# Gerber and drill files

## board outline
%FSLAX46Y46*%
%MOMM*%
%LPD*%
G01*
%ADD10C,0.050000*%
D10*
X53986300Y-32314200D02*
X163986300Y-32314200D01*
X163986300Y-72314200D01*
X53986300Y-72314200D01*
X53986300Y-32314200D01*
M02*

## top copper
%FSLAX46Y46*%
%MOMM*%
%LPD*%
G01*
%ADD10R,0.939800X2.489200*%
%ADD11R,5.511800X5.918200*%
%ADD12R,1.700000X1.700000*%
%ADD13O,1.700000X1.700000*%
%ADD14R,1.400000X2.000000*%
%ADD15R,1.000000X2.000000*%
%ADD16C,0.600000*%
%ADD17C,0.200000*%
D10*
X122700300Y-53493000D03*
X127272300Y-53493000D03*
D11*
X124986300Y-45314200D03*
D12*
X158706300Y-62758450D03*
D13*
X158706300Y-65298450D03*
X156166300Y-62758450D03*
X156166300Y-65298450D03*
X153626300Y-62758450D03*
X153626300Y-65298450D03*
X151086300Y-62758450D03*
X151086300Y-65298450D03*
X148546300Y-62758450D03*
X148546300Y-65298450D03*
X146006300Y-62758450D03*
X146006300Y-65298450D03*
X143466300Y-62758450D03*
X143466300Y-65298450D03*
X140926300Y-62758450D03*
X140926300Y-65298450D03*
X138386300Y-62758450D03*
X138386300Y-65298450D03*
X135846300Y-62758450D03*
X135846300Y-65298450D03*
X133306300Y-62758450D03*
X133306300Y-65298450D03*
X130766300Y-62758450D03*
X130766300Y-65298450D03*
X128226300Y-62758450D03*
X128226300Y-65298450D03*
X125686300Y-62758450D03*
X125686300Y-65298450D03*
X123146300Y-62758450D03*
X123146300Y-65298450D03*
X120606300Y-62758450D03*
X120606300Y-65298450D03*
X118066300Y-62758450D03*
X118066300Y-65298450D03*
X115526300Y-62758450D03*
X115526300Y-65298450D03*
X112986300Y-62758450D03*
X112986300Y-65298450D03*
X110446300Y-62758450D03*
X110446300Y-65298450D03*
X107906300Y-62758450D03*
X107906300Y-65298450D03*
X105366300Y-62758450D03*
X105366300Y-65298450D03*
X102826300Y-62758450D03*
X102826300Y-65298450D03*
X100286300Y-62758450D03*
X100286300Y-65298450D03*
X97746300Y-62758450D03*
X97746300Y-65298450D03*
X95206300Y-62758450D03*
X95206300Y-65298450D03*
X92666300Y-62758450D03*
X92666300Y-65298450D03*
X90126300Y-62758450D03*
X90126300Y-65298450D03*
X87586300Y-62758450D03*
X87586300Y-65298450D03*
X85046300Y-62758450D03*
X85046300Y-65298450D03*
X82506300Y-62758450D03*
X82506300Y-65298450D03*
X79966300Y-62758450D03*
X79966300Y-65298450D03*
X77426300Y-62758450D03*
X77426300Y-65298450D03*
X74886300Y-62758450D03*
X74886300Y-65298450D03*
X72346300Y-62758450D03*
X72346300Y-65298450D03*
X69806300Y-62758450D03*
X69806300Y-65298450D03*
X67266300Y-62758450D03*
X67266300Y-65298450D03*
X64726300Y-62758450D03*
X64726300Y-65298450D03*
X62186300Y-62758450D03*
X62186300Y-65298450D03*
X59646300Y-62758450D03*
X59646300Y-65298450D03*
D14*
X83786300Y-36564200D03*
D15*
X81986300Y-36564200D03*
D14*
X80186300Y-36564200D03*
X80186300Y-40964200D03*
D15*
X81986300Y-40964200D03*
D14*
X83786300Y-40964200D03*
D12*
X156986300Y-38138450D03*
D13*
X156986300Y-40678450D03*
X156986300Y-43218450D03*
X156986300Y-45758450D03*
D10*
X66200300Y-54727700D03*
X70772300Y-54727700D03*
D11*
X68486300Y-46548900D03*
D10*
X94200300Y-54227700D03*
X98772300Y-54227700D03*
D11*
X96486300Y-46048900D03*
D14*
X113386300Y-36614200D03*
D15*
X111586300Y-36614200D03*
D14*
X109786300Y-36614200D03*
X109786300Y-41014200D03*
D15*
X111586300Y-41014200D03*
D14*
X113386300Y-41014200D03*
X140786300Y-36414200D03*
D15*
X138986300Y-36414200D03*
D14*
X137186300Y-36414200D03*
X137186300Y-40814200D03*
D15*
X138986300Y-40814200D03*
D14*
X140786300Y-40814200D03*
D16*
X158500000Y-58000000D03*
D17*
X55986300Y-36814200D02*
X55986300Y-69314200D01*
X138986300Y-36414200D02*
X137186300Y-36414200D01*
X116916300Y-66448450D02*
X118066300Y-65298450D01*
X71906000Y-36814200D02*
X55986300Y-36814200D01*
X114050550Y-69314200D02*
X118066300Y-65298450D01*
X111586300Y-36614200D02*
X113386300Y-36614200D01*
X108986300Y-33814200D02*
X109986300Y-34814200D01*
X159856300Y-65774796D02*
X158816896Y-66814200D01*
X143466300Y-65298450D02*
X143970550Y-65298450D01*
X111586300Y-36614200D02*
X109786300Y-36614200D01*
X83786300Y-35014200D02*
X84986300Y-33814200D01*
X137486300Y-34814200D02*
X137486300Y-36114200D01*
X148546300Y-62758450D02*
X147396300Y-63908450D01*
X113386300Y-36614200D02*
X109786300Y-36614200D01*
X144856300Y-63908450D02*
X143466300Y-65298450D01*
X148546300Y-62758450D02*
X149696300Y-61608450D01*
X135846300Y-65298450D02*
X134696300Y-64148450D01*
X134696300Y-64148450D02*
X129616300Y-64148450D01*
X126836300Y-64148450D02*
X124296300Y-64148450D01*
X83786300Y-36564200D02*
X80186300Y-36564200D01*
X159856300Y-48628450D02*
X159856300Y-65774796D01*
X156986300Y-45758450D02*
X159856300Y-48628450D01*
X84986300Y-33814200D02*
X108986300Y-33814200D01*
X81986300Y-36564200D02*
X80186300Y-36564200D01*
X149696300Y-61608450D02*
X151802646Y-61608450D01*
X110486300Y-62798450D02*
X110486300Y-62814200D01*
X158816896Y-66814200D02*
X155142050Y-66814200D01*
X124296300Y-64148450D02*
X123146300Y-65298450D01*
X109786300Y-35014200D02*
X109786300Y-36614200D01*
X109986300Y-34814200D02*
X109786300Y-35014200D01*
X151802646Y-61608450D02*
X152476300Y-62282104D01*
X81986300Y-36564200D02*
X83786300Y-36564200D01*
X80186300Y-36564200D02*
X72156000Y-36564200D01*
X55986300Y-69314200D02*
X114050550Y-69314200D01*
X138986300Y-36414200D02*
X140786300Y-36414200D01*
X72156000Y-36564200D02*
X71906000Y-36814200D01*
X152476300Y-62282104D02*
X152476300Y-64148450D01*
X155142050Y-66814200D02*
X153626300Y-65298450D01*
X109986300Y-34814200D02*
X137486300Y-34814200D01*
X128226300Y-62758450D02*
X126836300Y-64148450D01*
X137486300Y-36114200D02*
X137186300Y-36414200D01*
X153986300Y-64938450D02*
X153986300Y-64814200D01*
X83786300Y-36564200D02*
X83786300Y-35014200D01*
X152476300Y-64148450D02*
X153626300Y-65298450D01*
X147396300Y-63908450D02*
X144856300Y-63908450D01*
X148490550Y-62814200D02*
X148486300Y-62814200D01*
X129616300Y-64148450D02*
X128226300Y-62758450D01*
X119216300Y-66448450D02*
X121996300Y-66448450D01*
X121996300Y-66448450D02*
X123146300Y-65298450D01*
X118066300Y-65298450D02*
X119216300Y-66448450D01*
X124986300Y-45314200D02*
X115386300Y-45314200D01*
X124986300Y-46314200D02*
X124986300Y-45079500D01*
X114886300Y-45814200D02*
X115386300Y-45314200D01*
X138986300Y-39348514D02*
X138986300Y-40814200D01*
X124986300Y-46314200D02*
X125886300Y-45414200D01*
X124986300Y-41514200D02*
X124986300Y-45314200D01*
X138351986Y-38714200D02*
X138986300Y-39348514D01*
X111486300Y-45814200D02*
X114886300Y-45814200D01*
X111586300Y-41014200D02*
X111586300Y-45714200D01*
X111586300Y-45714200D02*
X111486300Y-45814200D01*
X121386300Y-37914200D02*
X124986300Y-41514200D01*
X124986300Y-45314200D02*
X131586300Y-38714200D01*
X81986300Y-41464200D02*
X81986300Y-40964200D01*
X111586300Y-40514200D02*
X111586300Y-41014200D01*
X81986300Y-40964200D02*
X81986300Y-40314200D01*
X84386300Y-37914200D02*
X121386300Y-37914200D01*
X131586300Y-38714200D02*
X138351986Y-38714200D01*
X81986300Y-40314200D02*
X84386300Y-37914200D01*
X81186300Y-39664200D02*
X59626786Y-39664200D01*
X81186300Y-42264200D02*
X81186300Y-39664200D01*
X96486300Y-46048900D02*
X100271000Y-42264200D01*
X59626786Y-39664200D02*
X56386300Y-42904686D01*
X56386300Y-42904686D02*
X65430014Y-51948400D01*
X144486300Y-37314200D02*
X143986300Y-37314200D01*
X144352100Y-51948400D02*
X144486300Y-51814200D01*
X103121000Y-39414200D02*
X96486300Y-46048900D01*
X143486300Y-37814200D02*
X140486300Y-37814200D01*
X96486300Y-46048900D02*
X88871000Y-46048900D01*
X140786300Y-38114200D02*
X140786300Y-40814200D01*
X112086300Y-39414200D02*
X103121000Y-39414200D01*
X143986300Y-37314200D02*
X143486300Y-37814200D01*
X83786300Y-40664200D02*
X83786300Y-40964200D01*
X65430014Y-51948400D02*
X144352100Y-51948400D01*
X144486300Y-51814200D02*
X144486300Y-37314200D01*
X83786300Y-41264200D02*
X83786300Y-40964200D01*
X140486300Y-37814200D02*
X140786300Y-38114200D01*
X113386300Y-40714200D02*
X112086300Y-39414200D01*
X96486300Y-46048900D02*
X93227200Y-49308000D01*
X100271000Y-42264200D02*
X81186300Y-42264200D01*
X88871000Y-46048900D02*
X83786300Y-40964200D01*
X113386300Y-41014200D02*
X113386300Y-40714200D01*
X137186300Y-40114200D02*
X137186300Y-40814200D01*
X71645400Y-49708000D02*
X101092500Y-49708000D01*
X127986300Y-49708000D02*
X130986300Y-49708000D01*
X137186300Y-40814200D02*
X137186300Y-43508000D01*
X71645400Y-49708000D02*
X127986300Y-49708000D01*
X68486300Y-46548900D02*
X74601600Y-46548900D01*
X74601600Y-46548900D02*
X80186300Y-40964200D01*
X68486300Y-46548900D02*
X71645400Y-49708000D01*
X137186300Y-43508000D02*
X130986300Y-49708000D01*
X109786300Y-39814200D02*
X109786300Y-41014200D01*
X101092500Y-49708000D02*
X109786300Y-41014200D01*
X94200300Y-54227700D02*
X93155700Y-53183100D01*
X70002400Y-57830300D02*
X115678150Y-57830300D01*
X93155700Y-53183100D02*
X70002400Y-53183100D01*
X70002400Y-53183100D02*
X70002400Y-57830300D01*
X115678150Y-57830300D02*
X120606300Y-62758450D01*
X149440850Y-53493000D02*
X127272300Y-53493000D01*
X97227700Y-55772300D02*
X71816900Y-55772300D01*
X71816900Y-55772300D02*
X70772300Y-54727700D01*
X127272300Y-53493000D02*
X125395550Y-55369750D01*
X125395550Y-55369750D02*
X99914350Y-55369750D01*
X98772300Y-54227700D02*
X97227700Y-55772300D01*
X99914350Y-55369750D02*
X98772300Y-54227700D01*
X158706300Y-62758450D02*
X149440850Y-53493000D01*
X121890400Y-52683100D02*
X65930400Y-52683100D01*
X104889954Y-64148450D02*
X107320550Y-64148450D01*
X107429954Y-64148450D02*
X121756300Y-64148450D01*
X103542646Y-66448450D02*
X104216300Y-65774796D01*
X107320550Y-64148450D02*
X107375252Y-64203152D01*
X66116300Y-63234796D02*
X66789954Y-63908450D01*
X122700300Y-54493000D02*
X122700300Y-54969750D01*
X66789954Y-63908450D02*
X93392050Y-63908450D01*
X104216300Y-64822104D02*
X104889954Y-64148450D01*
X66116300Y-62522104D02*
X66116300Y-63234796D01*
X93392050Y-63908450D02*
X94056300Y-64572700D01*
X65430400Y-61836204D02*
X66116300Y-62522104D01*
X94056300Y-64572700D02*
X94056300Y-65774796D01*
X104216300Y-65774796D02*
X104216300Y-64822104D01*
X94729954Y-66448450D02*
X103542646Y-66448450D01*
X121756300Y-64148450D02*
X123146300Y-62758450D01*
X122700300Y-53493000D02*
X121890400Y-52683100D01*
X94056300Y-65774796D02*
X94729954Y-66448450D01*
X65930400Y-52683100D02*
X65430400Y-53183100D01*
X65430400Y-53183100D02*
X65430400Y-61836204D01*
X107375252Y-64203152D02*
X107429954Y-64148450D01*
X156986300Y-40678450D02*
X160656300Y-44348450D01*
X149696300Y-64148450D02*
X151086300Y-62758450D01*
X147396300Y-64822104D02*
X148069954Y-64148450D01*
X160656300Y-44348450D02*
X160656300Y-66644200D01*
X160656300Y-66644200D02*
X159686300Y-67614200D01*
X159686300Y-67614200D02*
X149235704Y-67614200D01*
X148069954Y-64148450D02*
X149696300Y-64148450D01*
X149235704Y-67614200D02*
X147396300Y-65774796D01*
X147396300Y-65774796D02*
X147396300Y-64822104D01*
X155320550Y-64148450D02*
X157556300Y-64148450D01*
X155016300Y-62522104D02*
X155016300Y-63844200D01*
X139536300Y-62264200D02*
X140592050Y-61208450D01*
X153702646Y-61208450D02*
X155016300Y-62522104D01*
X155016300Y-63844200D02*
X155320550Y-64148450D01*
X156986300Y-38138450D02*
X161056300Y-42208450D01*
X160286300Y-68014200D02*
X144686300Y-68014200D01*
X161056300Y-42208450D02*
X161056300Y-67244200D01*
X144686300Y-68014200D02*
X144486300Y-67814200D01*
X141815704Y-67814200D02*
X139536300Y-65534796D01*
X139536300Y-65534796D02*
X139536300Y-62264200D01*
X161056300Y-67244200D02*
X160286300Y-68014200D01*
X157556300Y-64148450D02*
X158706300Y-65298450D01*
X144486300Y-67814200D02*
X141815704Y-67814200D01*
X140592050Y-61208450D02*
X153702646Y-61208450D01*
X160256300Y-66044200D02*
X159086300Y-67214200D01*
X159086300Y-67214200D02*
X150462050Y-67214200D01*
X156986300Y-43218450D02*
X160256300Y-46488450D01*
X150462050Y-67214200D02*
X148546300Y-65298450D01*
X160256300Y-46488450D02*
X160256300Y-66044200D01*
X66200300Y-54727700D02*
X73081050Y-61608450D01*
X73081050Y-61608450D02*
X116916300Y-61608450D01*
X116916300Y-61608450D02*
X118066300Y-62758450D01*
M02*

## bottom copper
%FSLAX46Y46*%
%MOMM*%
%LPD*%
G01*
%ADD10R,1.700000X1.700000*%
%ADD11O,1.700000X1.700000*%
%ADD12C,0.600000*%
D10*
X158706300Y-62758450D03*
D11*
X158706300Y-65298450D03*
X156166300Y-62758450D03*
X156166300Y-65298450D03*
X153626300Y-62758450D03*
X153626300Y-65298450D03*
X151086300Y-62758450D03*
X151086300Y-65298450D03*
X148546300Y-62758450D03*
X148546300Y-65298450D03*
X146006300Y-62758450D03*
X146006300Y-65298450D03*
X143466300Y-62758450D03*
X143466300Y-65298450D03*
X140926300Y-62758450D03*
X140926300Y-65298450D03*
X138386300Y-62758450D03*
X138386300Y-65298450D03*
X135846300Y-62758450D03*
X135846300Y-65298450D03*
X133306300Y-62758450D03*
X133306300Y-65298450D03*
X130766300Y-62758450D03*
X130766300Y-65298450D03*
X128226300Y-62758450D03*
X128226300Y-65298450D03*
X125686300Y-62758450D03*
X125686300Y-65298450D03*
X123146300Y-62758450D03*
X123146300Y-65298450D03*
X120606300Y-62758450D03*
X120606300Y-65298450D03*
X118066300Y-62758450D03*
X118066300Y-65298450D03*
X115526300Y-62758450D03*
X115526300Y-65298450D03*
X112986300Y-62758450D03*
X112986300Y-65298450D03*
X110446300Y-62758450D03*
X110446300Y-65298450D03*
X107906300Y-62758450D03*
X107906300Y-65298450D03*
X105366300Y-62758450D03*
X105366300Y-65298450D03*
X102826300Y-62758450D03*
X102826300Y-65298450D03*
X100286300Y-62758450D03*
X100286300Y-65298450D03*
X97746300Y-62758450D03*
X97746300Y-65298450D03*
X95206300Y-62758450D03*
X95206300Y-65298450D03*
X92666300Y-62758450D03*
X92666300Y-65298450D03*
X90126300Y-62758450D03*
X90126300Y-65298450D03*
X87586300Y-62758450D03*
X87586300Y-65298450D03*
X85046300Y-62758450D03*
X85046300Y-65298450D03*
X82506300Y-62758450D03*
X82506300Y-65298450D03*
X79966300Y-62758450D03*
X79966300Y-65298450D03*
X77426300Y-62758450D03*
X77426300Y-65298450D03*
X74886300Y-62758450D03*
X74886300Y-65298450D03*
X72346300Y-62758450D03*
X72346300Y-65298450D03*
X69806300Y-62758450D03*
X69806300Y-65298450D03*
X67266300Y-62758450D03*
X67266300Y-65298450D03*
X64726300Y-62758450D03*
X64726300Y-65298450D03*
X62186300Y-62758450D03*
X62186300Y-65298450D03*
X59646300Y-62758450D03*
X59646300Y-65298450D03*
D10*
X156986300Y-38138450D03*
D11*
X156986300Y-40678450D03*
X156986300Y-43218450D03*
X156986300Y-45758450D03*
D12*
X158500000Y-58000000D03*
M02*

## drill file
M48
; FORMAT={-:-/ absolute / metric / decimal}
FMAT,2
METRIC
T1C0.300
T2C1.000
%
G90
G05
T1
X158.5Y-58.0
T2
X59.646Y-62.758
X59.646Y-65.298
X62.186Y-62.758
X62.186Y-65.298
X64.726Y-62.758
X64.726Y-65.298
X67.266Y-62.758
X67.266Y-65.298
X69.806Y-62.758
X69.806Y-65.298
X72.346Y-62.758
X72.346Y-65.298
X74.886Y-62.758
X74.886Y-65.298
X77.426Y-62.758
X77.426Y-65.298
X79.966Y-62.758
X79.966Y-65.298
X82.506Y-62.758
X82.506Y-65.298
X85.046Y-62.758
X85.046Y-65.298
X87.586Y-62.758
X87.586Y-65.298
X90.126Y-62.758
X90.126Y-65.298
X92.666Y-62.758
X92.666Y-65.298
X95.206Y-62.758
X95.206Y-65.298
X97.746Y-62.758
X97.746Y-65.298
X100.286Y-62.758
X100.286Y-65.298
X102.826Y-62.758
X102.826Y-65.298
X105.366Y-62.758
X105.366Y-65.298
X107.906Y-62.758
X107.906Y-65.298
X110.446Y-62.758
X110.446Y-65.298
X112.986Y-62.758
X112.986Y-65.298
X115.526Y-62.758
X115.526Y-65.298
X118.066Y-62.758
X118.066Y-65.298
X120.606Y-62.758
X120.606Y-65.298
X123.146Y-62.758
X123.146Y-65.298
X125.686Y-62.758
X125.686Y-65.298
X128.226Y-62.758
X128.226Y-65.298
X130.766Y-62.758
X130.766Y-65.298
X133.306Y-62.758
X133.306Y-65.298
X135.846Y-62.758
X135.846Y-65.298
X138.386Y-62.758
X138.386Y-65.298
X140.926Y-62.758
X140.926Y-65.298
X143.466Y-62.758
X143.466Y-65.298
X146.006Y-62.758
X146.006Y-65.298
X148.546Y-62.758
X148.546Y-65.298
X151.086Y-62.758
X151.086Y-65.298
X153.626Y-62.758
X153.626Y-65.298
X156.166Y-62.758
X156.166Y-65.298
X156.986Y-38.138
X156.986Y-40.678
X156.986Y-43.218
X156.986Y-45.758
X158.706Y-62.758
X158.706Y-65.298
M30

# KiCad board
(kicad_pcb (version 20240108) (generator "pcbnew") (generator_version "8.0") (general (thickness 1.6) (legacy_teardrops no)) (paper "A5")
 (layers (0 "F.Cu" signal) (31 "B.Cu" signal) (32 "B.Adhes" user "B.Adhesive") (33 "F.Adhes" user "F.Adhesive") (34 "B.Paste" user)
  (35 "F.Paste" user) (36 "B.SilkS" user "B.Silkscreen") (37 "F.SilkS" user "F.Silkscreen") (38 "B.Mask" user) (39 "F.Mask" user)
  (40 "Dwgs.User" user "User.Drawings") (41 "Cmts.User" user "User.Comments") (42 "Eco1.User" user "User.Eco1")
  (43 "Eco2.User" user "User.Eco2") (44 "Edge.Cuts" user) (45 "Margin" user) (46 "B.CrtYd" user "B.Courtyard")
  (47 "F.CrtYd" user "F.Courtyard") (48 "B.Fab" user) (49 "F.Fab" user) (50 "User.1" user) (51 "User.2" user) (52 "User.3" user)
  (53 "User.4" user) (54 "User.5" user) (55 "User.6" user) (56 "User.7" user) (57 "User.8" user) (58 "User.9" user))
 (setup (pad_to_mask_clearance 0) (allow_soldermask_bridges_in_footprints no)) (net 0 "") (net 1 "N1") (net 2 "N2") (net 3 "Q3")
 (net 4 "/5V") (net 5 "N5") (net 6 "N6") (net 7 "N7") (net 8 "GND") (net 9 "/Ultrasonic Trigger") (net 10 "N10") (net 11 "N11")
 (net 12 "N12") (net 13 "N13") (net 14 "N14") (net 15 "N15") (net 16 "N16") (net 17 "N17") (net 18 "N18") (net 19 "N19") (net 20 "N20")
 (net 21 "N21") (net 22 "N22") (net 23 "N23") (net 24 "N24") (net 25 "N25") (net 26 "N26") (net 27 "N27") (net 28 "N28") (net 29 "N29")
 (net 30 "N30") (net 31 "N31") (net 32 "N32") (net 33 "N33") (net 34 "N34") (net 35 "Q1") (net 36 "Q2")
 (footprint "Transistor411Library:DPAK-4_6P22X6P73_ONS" (layer "F.Cu") (at 124.9863 47.0795)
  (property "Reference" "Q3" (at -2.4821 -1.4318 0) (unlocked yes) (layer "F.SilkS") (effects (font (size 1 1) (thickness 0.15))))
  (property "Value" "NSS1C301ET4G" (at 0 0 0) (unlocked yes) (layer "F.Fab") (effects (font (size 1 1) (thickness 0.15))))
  (pad "1" smd rect (at -2.286 6.4135) (size 0.9398 2.4892) (layers "F.Cu" "F.Paste" "F.Mask") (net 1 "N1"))
  (pad "2" smd rect (at 2.286 6.4135) (size 0.9398 2.4892) (layers "F.Cu" "F.Paste" "F.Mask") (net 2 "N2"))
  (pad "3" smd rect (at 0 -1.7653) (size 5.5118 5.9182) (layers "F.Cu" "F.Paste" "F.Mask") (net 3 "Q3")))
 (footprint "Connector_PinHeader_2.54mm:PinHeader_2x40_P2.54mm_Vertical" (layer "F.Cu") (at 158.7063 62.75845 -90)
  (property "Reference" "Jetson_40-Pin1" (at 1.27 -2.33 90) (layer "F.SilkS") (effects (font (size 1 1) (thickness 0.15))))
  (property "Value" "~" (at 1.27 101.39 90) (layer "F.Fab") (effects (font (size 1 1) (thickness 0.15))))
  (pad "1" thru_hole rect (at 0 0 270) (size 1.7 1.7) (drill 1) (layers "*.Cu" "*.Mask") (remove_unused_layers no) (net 2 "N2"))
  (pad "2" thru_hole oval (at 2.54 0 270) (size 1.7 1.7) (drill 1) (layers "*.Cu" "*.Mask") (remove_unused_layers no) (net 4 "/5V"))
  (pad "3" thru_hole oval (at 0 2.54 270) (size 1.7 1.7) (drill 1) (layers "*.Cu" "*.Mask") (remove_unused_layers no) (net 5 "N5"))
  (pad "4" thru_hole oval (at 2.54 2.54 270) (size 1.7 1.7) (drill 1) (layers "*.Cu" "*.Mask") (remove_unused_layers no) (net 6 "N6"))
  (pad "5" thru_hole oval (at 0 5.08 270) (size 1.7 1.7) (drill 1) (layers "*.Cu" "*.Mask") (remove_unused_layers no) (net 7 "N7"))
  (pad "6" thru_hole oval (at 2.54 5.08 270) (size 1.7 1.7) (drill 1) (layers "*.Cu" "*.Mask") (remove_unused_layers no) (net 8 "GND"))
  (pad "7" thru_hole oval (at 0 7.62 270) (size 1.7 1.7) (drill 1) (layers "*.Cu" "*.Mask") (remove_unused_layers no)
   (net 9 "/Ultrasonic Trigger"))
  (pad "8" thru_hole oval (at 2.54 7.62 270) (size 1.7 1.7) (drill 1) (layers "*.Cu" "*.Mask") (remove_unused_layers no) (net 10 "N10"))
  (pad "9" thru_hole oval (at 0 10.16 270) (size 1.7 1.7) (drill 1) (layers "*.Cu" "*.Mask") (remove_unused_layers no) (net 8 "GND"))
  (pad "10" thru_hole oval (at 2.54 10.16 270) (size 1.7 1.7) (drill 1) (layers "*.Cu" "*.Mask") (remove_unused_layers no) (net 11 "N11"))
  (pad "11" thru_hole oval (at 0 12.7 270) (size 1.7 1.7) (drill 1) (layers "*.Cu" "*.Mask") (remove_unused_layers no) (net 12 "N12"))
  (pad "12" thru_hole oval (at 2.54 12.7 270) (size 1.7 1.7) (drill 1) (layers "*.Cu" "*.Mask") (remove_unused_layers no) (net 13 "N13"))
  (pad "13" thru_hole oval (at 0 15.24 270) (size 1.7 1.7) (drill 1) (layers "*.Cu" "*.Mask") (remove_unused_layers no) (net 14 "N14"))
  (pad "14" thru_hole oval (at 2.54 15.24 270) (size 1.7 1.7) (drill 1) (layers "*.Cu" "*.Mask") (remove_unused_layers no) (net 8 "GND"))
  (pad "15" thru_hole oval (at 0 17.78 270) (size 1.7 1.7) (drill 1) (layers "*.Cu" "*.Mask") (remove_unused_layers no) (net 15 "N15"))
  (pad "16" thru_hole oval (at 2.54 17.78 270) (size 1.7 1.7) (drill 1) (layers "*.Cu" "*.Mask") (remove_unused_layers no) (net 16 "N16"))
  (pad "17" thru_hole oval (at 0 20.32 270) (size 1.7 1.7) (drill 1) (layers "*.Cu" "*.Mask") (remove_unused_layers no) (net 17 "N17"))
  (pad "18" thru_hole oval (at 2.54 20.32 270) (size 1.7 1.7) (drill 1) (layers "*.Cu" "*.Mask") (remove_unused_layers no) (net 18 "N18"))
  (pad "19" thru_hole oval (at 0 22.86 270) (size 1.7 1.7) (drill 1) (layers "*.Cu" "*.Mask") (remove_unused_layers no) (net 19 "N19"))
  (pad "20" thru_hole oval (at 2.54 22.86 270) (size 1.7 1.7) (drill 1) (layers "*.Cu" "*.Mask") (remove_unused_layers no) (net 8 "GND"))
  (pad "21" thru_hole oval (at 0 25.4 270) (size 1.7 1.7) (drill 1) (layers "*.Cu" "*.Mask") (remove_unused_layers no) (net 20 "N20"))
  (pad "22" thru_hole oval (at 2.54 25.4 270) (size 1.7 1.7) (drill 1) (layers "*.Cu" "*.Mask") (remove_unused_layers no) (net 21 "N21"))
  (pad "23" thru_hole oval (at 0 27.94 270) (size 1.7 1.7) (drill 1) (layers "*.Cu" "*.Mask") (remove_unused_layers no) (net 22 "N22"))
  (pad "24" thru_hole oval (at 2.54 27.94 270) (size 1.7 1.7) (drill 1) (layers "*.Cu" "*.Mask") (remove_unused_layers no) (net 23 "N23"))
  (pad "25" thru_hole oval (at 0 30.48 270) (size 1.7 1.7) (drill 1) (layers "*.Cu" "*.Mask") (remove_unused_layers no) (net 8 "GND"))
  (pad "26" thru_hole oval (at 2.54 30.48 270) (size 1.7 1.7) (drill 1) (layers "*.Cu" "*.Mask") (remove_unused_layers no) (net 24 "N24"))
  (pad "27" thru_hole oval (at 0 33.02 270) (size 1.7 1.7) (drill 1) (layers "*.Cu" "*.Mask") (remove_unused_layers no) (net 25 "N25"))
  (pad "28" thru_hole oval (at 2.54 33.02 270) (size 1.7 1.7) (drill 1) (layers "*.Cu" "*.Mask") (remove_unused_layers no) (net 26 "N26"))
  (pad "29" thru_hole oval (at 0 35.56 270) (size 1.7 1.7) (drill 1) (layers "*.Cu" "*.Mask") (remove_unused_layers no) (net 1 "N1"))
  (pad "30" thru_hole oval (at 2.54 35.56 270) (size 1.7 1.7) (drill 1) (layers "*.Cu" "*.Mask") (remove_unused_layers no) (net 8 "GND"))
  (pad "31" thru_hole oval (at 0 38.1 270) (size 1.7 1.7) (drill 1) (layers "*.Cu" "*.Mask") (remove_unused_layers no) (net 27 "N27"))
  (pad "32" thru_hole oval (at 2.54 38.1 270) (size 1.7 1.7) (drill 1) (layers "*.Cu" "*.Mask") (remove_unused_layers no) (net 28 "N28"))
  (pad "33" thru_hole oval (at 0 40.64 270) (size 1.7 1.7) (drill 1) (layers "*.Cu" "*.Mask") (remove_unused_layers no) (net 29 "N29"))
  (pad "34" thru_hole oval (at 2.54 40.64 270) (size 1.7 1.7) (drill 1) (layers "*.Cu" "*.Mask") (remove_unused_layers no) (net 8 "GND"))
  (pad "35" thru_hole oval (at 0 43.18 270) (size 1.7 1.7) (drill 1) (layers "*.Cu" "*.Mask") (remove_unused_layers no) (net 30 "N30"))
  (pad "36" thru_hole oval (at 2.54 43.18 270) (size 1.7 1.7) (drill 1) (layers "*.Cu" "*.Mask") (remove_unused_layers no) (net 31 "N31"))
  (pad "37" thru_hole oval (at 0 45.72 270) (size 1.7 1.7) (drill 1) (layers "*.Cu" "*.Mask") (remove_unused_layers no) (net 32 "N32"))
  (pad "38" thru_hole oval (at 2.54 45.72 270) (size 1.7 1.7) (drill 1) (layers "*.Cu" "*.Mask") (remove_unused_layers no) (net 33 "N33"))
  (pad "39" thru_hole oval (at 0 48.26 270) (size 1.7 1.7) (drill 1) (layers "*.Cu" "*.Mask") (remove_unused_layers no) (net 8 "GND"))
  (pad "40" thru_hole oval (at 2.54 48.26 270) (size 1.7 1.7) (drill 1) (layers "*.Cu" "*.Mask") (remove_unused_layers no) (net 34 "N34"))
  (pad "41" thru_hole oval (at 0 50.8 270) (size 1.7 1.7) (drill 1) (layers "*.Cu" "*.Mask") (remove_unused_layers no))
  (pad "42" thru_hole oval (at 2.54 50.8 270) (size 1.7 1.7) (drill 1) (layers "*.Cu" "*.Mask") (remove_unused_layers no))
  (pad "43" thru_hole oval (at 0 53.34 270) (size 1.7 1.7) (drill 1) (layers "*.Cu" "*.Mask") (remove_unused_layers no))
  (pad "44" thru_hole oval (at 2.54 53.34 270) (size 1.7 1.7) (drill 1) (layers "*.Cu" "*.Mask") (remove_unused_layers no))
  (pad "45" thru_hole oval (at 0 55.88 270) (size 1.7 1.7) (drill 1) (layers "*.Cu" "*.Mask") (remove_unused_layers no))
  (pad "46" thru_hole oval (at 2.54 55.88 270) (size 1.7 1.7) (drill 1) (layers "*.Cu" "*.Mask") (remove_unused_layers no))
  (pad "47" thru_hole oval (at 0 58.42 270) (size 1.7 1.7) (drill 1) (layers "*.Cu" "*.Mask") (remove_unused_layers no))
  (pad "48" thru_hole oval (at 2.54 58.42 270) (size 1.7 1.7) (drill 1) (layers "*.Cu" "*.Mask") (remove_unused_layers no))
  (pad "49" thru_hole oval (at 0 60.96 270) (size 1.7 1.7) (drill 1) (layers "*.Cu" "*.Mask") (remove_unused_layers no))
  (pad "50" thru_hole oval (at 2.54 60.96 270) (size 1.7 1.7) (drill 1) (layers "*.Cu" "*.Mask") (remove_unused_layers no))
  (pad "51" thru_hole oval (at 0 63.5 270) (size 1.7 1.7) (drill 1) (layers "*.Cu" "*.Mask") (remove_unused_layers no))
  (pad "52" thru_hole oval (at 2.54 63.5 270) (size 1.7 1.7) (drill 1) (layers "*.Cu" "*.Mask") (remove_unused_layers no))
  (pad "53" thru_hole oval (at 0 66.04 270) (size 1.7 1.7) (drill 1) (layers "*.Cu" "*.Mask") (remove_unused_layers no))
  (pad "54" thru_hole oval (at 2.54 66.04 270) (size 1.7 1.7) (drill 1) (layers "*.Cu" "*.Mask") (remove_unused_layers no))
  (pad "55" thru_hole oval (at 0 68.58 270) (size 1.7 1.7) (drill 1) (layers "*.Cu" "*.Mask") (remove_unused_layers no))
  (pad "56" thru_hole oval (at 2.54 68.58 270) (size 1.7 1.7) (drill 1) (layers "*.Cu" "*.Mask") (remove_unused_layers no))
  (pad "57" thru_hole oval (at 0 71.12 270) (size 1.7 1.7) (drill 1) (layers "*.Cu" "*.Mask") (remove_unused_layers no))
  (pad "58" thru_hole oval (at 2.54 71.12 270) (size 1.7 1.7) (drill 1) (layers "*.Cu" "*.Mask") (remove_unused_layers no))
  (pad "59" thru_hole oval (at 0 73.66 270) (size 1.7 1.7) (drill 1) (layers "*.Cu" "*.Mask") (remove_unused_layers no))
  (pad "60" thru_hole oval (at 2.54 73.66 270) (size 1.7 1.7) (drill 1) (layers "*.Cu" "*.Mask") (remove_unused_layers no))
  (pad "61" thru_hole oval (at 0 76.2 270) (size 1.7 1.7) (drill 1) (layers "*.Cu" "*.Mask") (remove_unused_layers no))
  (pad "62" thru_hole oval (at 2.54 76.2 270) (size 1.7 1.7) (drill 1) (layers "*.Cu" "*.Mask") (remove_unused_layers no))
  (pad "63" thru_hole oval (at 0 78.74 270) (size 1.7 1.7) (drill 1) (layers "*.Cu" "*.Mask") (remove_unused_layers no))
  (pad "64" thru_hole oval (at 2.54 78.74 270) (size 1.7 1.7) (drill 1) (layers "*.Cu" "*.Mask") (remove_unused_layers no))
  (pad "65" thru_hole oval (at 0 81.28 270) (size 1.7 1.7) (drill 1) (layers "*.Cu" "*.Mask") (remove_unused_layers no))
  (pad "66" thru_hole oval (at 2.54 81.28 270) (size 1.7 1.7) (drill 1) (layers "*.Cu" "*.Mask") (remove_unused_layers no))
  (pad "67" thru_hole oval (at 0 83.82 270) (size 1.7 1.7) (drill 1) (layers "*.Cu" "*.Mask") (remove_unused_layers no))
  (pad "68" thru_hole oval (at 2.54 83.82 270) (size 1.7 1.7) (drill 1) (layers "*.Cu" "*.Mask") (remove_unused_layers no))
  (pad "69" thru_hole oval (at 0 86.36 270) (size 1.7 1.7) (drill 1) (layers "*.Cu" "*.Mask") (remove_unused_layers no))
  (pad "70" thru_hole oval (at 2.54 86.36 270) (size 1.7 1.7) (drill 1) (layers "*.Cu" "*.Mask") (remove_unused_layers no))
  (pad "71" thru_hole oval (at 0 88.9 270) (size 1.7 1.7) (drill 1) (layers "*.Cu" "*.Mask") (remove_unused_layers no))
  (pad "72" thru_hole oval (at 2.54 88.9 270) (size 1.7 1.7) (drill 1) (layers "*.Cu" "*.Mask") (remove_unused_layers no))
  (pad "73" thru_hole oval (at 0 91.44 270) (size 1.7 1.7) (drill 1) (layers "*.Cu" "*.Mask") (remove_unused_layers no))
  (pad "74" thru_hole oval (at 2.54 91.44 270) (size 1.7 1.7) (drill 1) (layers "*.Cu" "*.Mask") (remove_unused_layers no))
  (pad "75" thru_hole oval (at 0 93.98 270) (size 1.7 1.7) (drill 1) (layers "*.Cu" "*.Mask") (remove_unused_layers no))
  (pad "76" thru_hole oval (at 2.54 93.98 270) (size 1.7 1.7) (drill 1) (layers "*.Cu" "*.Mask") (remove_unused_layers no))
  (pad "77" thru_hole oval (at 0 96.52 270) (size 1.7 1.7) (drill 1) (layers "*.Cu" "*.Mask") (remove_unused_layers no))
  (pad "78" thru_hole oval (at 2.54 96.52 270) (size 1.7 1.7) (drill 1) (layers "*.Cu" "*.Mask") (remove_unused_layers no))
  (pad "79" thru_hole oval (at 0 99.06 270) (size 1.7 1.7) (drill 1) (layers "*.Cu" "*.Mask") (remove_unused_layers no))
  (pad "80" thru_hole oval (at 2.54 99.06 270) (size 1.7 1.7) (drill 1) (layers "*.Cu" "*.Mask") (remove_unused_layers no)))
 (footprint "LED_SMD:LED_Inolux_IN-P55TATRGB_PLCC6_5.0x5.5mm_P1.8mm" (layer "F.Cu") (at 81.9863 38.7642 -90)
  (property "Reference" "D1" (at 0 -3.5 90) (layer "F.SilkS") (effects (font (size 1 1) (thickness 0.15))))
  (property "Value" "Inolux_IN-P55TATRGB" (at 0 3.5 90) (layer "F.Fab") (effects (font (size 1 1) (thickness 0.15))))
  (pad "1" smd rect (at -2.2 -1.8 270) (size 2 1.4) (layers "F.Cu" "F.Paste" "F.Mask") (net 8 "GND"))
  (pad "2" smd rect (at -2.2 0 270) (size 2 1) (layers "F.Cu" "F.Paste" "F.Mask") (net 8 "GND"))
  (pad "3" smd rect (at -2.2 1.8 270) (size 2 1.4) (layers "F.Cu" "F.Paste" "F.Mask") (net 8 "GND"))
  (pad "4" smd rect (at 2.2 1.8 270) (size 2 1.4) (layers "F.Cu" "F.Paste" "F.Mask") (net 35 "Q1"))
  (pad "5" smd rect (at 2.2 0 270) (size 2 1) (layers "F.Cu" "F.Paste" "F.Mask") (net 3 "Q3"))
  (pad "6" smd rect (at 2.2 -1.8 270) (size 2 1.4) (layers "F.Cu" "F.Paste" "F.Mask") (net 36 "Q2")))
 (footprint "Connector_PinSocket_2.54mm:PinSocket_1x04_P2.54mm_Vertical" (layer "F.Cu") (at 156.9863 38.13845)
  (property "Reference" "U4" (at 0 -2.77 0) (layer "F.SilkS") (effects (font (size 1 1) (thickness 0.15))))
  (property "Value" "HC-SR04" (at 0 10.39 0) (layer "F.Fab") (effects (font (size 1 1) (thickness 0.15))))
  (pad "1" thru_hole rect (at 0 0) (size 1.7 1.7) (drill 1) (layers "*.Cu" "*.Mask") (remove_unused_layers no) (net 4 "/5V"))
  (pad "2" thru_hole oval (at 0 2.54) (size 1.7 1.7) (drill 1) (layers "*.Cu" "*.Mask") (remove_unused_layers no)
   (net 9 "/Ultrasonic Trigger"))
  (pad "3" thru_hole oval (at 0 5.08) (size 1.7 1.7) (drill 1) (layers "*.Cu" "*.Mask") (remove_unused_layers no) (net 11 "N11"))
  (pad "4" thru_hole oval (at 0 7.62) (size 1.7 1.7) (drill 1) (layers "*.Cu" "*.Mask") (remove_unused_layers no) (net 8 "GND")))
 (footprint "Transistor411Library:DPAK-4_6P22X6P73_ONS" (layer "F.Cu") (at 68.4863 48.3142)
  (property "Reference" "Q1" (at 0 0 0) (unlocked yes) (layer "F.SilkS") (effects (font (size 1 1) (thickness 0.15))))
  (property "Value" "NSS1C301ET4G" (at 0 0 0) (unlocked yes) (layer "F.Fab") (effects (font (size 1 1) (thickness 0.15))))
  (pad "1" smd rect (at -2.286 6.4135) (size 0.9398 2.4892) (layers "F.Cu" "F.Paste" "F.Mask") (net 29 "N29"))
  (pad "2" smd rect (at 2.286 6.4135) (size 0.9398 2.4892) (layers "F.Cu" "F.Paste" "F.Mask") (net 2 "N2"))
  (pad "3" smd rect (at 0 -1.7653) (size 5.5118 5.9182) (layers "F.Cu" "F.Paste" "F.Mask") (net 35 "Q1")))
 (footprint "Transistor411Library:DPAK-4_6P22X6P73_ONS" (layer "F.Cu") (at 96.4863 47.8142)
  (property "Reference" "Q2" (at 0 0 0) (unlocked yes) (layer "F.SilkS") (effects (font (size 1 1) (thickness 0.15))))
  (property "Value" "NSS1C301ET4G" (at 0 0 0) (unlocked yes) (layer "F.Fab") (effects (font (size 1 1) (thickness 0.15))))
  (pad "1" smd rect (at -2.286 6.4135) (size 0.9398 2.4892) (layers "F.Cu" "F.Paste" "F.Mask") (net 27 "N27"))
  (pad "2" smd rect (at 2.286 6.4135) (size 0.9398 2.4892) (layers "F.Cu" "F.Paste" "F.Mask") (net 2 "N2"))
  (pad "3" smd rect (at 0 -1.7653) (size 5.5118 5.9182) (layers "F.Cu" "F.Paste" "F.Mask") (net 36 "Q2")))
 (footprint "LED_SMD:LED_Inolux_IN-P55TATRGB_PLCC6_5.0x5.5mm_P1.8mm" (layer "F.Cu") (at 111.5863 38.8142 -90)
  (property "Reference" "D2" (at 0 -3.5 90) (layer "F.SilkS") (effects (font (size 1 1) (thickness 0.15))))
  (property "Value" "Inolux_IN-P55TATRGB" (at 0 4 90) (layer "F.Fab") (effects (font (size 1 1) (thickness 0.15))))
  (pad "1" smd rect (at -2.2 -1.8 270) (size 2 1.4) (layers "F.Cu" "F.Paste" "F.Mask") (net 8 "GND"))
  (pad "2" smd rect (at -2.2 0 270) (size 2 1) (layers "F.Cu" "F.Paste" "F.Mask") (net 8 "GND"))
  (pad "3" smd rect (at -2.2 1.8 270) (size 2 1.4) (layers "F.Cu" "F.Paste" "F.Mask") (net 8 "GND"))
  (pad "4" smd rect (at 2.2 1.8 270) (size 2 1.4) (layers "F.Cu" "F.Paste" "F.Mask") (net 35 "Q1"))
  (pad "5" smd rect (at 2.2 0 270) (size 2 1) (layers "F.Cu" "F.Paste" "F.Mask") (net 3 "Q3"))
  (pad "6" smd rect (at 2.2 -1.8 270) (size 2 1.4) (layers "F.Cu" "F.Paste" "F.Mask") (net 36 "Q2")))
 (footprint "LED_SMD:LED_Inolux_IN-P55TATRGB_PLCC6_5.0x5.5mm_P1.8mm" (layer "F.Cu") (at 138.9863 38.6142 -90)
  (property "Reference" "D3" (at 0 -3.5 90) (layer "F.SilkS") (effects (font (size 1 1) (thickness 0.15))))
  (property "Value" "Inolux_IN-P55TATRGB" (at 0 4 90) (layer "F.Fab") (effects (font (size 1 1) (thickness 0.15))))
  (pad "1" smd rect (at -2.2 -1.8 270) (size 2 1.4) (layers "F.Cu" "F.Paste" "F.Mask") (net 8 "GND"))
  (pad "2" smd rect (at -2.2 0 270) (size 2 1) (layers "F.Cu" "F.Paste" "F.Mask") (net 8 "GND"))
  (pad "3" smd rect (at -2.2 1.8 270) (size 2 1.4) (layers "F.Cu" "F.Paste" "F.Mask") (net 8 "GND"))
  (pad "4" smd rect (at 2.2 1.8 270) (size 2 1.4) (layers "F.Cu" "F.Paste" "F.Mask") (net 35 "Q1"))
  (pad "5" smd rect (at 2.2 0 270) (size 2 1) (layers "F.Cu" "F.Paste" "F.Mask") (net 3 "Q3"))
  (pad "6" smd rect (at 2.2 -1.8 270) (size 2 1.4) (layers "F.Cu" "F.Paste" "F.Mask") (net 36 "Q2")))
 (gr_rect (start 53.9863 32.3142) (end 163.9863 72.3142) (stroke (width 0.05) (type default)) (fill none) (layer "Edge.Cuts"))
 (via (at 158.5 58) (size 0.6) (drill 0.3) (layers "F.Cu" "B.Cu") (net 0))
 (segment (start 55.9863 36.8142) (end 55.9863 69.3142) (width 0.2) (layer "F.Cu") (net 8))
 (segment (start 138.9863 36.4142) (end 137.1863 36.4142) (width 0.2) (layer "F.Cu") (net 8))
 (segment (start 116.9163 66.44845) (end 118.0663 65.29845) (width 0.2) (layer "F.Cu") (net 8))
 (segment (start 71.906 36.8142) (end 55.9863 36.8142) (width 0.2) (layer "F.Cu") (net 8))
 (segment (start 114.05055 69.3142) (end 118.0663 65.29845) (width 0.2) (layer "F.Cu") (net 8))
 (segment (start 111.5863 36.6142) (end 113.3863 36.6142) (width 0.2) (layer "F.Cu") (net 8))
 (segment (start 108.9863 33.8142) (end 109.9863 34.8142) (width 0.2) (layer "F.Cu") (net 8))
 (segment (start 159.8563 65.774796) (end 158.816896 66.8142) (width 0.2) (layer "F.Cu") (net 8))
 (segment (start 143.4663 65.29845) (end 143.97055 65.29845) (width 0.2) (layer "F.Cu") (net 8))
 (segment (start 111.5863 36.6142) (end 109.7863 36.6142) (width 0.2) (layer "F.Cu") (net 8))
 (segment (start 83.7863 35.0142) (end 84.9863 33.8142) (width 0.2) (layer "F.Cu") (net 8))
 (segment (start 137.4863 34.8142) (end 137.4863 36.1142) (width 0.2) (layer "F.Cu") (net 8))
 (segment (start 148.5463 62.75845) (end 147.3963 63.90845) (width 0.2) (layer "F.Cu") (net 8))
 (segment (start 113.3863 36.6142) (end 109.7863 36.6142) (width 0.2) (layer "F.Cu") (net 8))
 (segment (start 144.8563 63.90845) (end 143.4663 65.29845) (width 0.2) (layer "F.Cu") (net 8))
 (segment (start 148.5463 62.75845) (end 149.6963 61.60845) (width 0.2) (layer "F.Cu") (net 8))
 (segment (start 135.8463 65.29845) (end 134.6963 64.14845) (width 0.2) (layer "F.Cu") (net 8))
 (segment (start 134.6963 64.14845) (end 129.6163 64.14845) (width 0.2) (layer "F.Cu") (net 8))
 (segment (start 126.8363 64.14845) (end 124.2963 64.14845) (width 0.2) (layer "F.Cu") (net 8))
 (segment (start 83.7863 36.5642) (end 80.1863 36.5642) (width 0.2) (layer "F.Cu") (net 8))
 (segment (start 159.8563 48.62845) (end 159.8563 65.774796) (width 0.2) (layer "F.Cu") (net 8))
 (segment (start 156.9863 45.75845) (end 159.8563 48.62845) (width 0.2) (layer "F.Cu") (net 8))
 (segment (start 84.9863 33.8142) (end 108.9863 33.8142) (width 0.2) (layer "F.Cu") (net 8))
 (segment (start 81.9863 36.5642) (end 80.1863 36.5642) (width 0.2) (layer "F.Cu") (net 8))
 (segment (start 149.6963 61.60845) (end 151.802646 61.60845) (width 0.2) (layer "F.Cu") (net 8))
 (segment (start 110.4863 62.79845) (end 110.4863 62.8142) (width 0.2) (layer "F.Cu") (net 8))
 (segment (start 158.816896 66.8142) (end 155.14205 66.8142) (width 0.2) (layer "F.Cu") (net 8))
 (segment (start 124.2963 64.14845) (end 123.1463 65.29845) (width 0.2) (layer "F.Cu") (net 8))
 (segment (start 109.7863 35.0142) (end 109.7863 36.6142) (width 0.2) (layer "F.Cu") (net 8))
 (segment (start 109.9863 34.8142) (end 109.7863 35.0142) (width 0.2) (layer "F.Cu") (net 8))
 (segment (start 151.802646 61.60845) (end 152.4763 62.282104) (width 0.2) (layer "F.Cu") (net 8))
 (segment (start 81.9863 36.5642) (end 83.7863 36.5642) (width 0.2) (layer "F.Cu") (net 8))
 (segment (start 80.1863 36.5642) (end 72.156 36.5642) (width 0.2) (layer "F.Cu") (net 8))
 (segment (start 55.9863 69.3142) (end 114.05055 69.3142) (width 0.2) (layer "F.Cu") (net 8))
 (segment (start 138.9863 36.4142) (end 140.7863 36.4142) (width 0.2) (layer "F.Cu") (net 8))
 (segment (start 72.156 36.5642) (end 71.906 36.8142) (width 0.2) (layer "F.Cu") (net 8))
 (segment (start 152.4763 62.282104) (end 152.4763 64.14845) (width 0.2) (layer "F.Cu") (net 8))
 (segment (start 155.14205 66.8142) (end 153.6263 65.29845) (width 0.2) (layer "F.Cu") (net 8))
 (segment (start 109.9863 34.8142) (end 137.4863 34.8142) (width 0.2) (layer "F.Cu") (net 8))
 (segment (start 128.2263 62.75845) (end 126.8363 64.14845) (width 0.2) (layer "F.Cu") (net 8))
 (segment (start 137.4863 36.1142) (end 137.1863 36.4142) (width 0.2) (layer "F.Cu") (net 8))
 (segment (start 153.9863 64.93845) (end 153.9863 64.8142) (width 0.2) (layer "F.Cu") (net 8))
 (segment (start 83.7863 36.5642) (end 83.7863 35.0142) (width 0.2) (layer "F.Cu") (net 8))
 (segment (start 152.4763 64.14845) (end 153.6263 65.29845) (width 0.2) (layer "F.Cu") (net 8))
 (segment (start 147.3963 63.90845) (end 144.8563 63.90845) (width 0.2) (layer "F.Cu") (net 8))
 (segment (start 148.49055 62.8142) (end 148.4863 62.8142) (width 0.2) (layer "F.Cu") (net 8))
 (segment (start 129.6163 64.14845) (end 128.2263 62.75845) (width 0.2) (layer "F.Cu") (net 8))
 (segment (start 119.2163 66.44845) (end 121.9963 66.44845) (width 0.2) (layer "F.Cu") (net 8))
 (segment (start 121.9963 66.44845) (end 123.1463 65.29845) (width 0.2) (layer "F.Cu") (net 8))
 (segment (start 118.0663 65.29845) (end 119.2163 66.44845) (width 0.2) (layer "F.Cu") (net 8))
 (segment (start 124.9863 45.3142) (end 115.3863 45.3142) (width 0.2) (layer "F.Cu") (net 3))
 (segment (start 124.9863 46.3142) (end 124.9863 45.0795) (width 0.2) (layer "F.Cu") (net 3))
 (segment (start 114.8863 45.8142) (end 115.3863 45.3142) (width 0.2) (layer "F.Cu") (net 3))
 (segment (start 138.9863 39.348514) (end 138.9863 40.8142) (width 0.2) (layer "F.Cu") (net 3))
 (segment (start 124.9863 46.3142) (end 125.8863 45.4142) (width 0.2) (layer "F.Cu") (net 3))
 (segment (start 124.9863 41.5142) (end 124.9863 45.3142) (width 0.2) (layer "F.Cu") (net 3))
 (segment (start 138.351986 38.7142) (end 138.9863 39.348514) (width 0.2) (layer "F.Cu") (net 3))
 (segment (start 111.4863 45.8142) (end 114.8863 45.8142) (width 0.2) (layer "F.Cu") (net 3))
 (segment (start 111.5863 41.0142) (end 111.5863 45.7142) (width 0.2) (layer "F.Cu") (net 3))
 (segment (start 111.5863 45.7142) (end 111.4863 45.8142) (width 0.2) (layer "F.Cu") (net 3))
 (segment (start 121.3863 37.9142) (end 124.9863 41.5142) (width 0.2) (layer "F.Cu") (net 3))
 (segment (start 124.9863 45.3142) (end 131.5863 38.7142) (width 0.2) (layer "F.Cu") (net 3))
 (segment (start 81.9863 41.4642) (end 81.9863 40.9642) (width 0.2) (layer "F.Cu") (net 3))
 (segment (start 111.5863 40.5142) (end 111.5863 41.0142) (width 0.2) (layer "F.Cu") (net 3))
 (segment (start 81.9863 40.9642) (end 81.9863 40.3142) (width 0.2) (layer "F.Cu") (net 3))
 (segment (start 84.3863 37.9142) (end 121.3863 37.9142) (width 0.2) (layer "F.Cu") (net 3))
 (segment (start 131.5863 38.7142) (end 138.351986 38.7142) (width 0.2) (layer "F.Cu") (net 3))
 (segment (start 81.9863 40.3142) (end 84.3863 37.9142) (width 0.2) (layer "F.Cu") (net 3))
 (segment (start 81.1863 39.6642) (end 59.626786 39.6642) (width 0.2) (layer "F.Cu") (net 36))
 (segment (start 81.1863 42.2642) (end 81.1863 39.6642) (width 0.2) (layer "F.Cu") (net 36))
 (segment (start 96.4863 46.0489) (end 100.271 42.2642) (width 0.2) (layer "F.Cu") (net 36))
 (segment (start 59.626786 39.6642) (end 56.3863 42.904686) (width 0.2) (layer "F.Cu") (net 36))
 (segment (start 56.3863 42.904686) (end 65.430014 51.9484) (width 0.2) (layer "F.Cu") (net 36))
 (segment (start 144.4863 37.3142) (end 143.9863 37.3142) (width 0.2) (layer "F.Cu") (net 36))
 (segment (start 144.3521 51.9484) (end 144.4863 51.8142) (width 0.2) (layer "F.Cu") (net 36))
 (segment (start 103.121 39.4142) (end 96.4863 46.0489) (width 0.2) (layer "F.Cu") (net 36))
 (segment (start 143.4863 37.8142) (end 140.4863 37.8142) (width 0.2) (layer "F.Cu") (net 36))
 (segment (start 96.4863 46.0489) (end 88.871 46.0489) (width 0.2) (layer "F.Cu") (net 36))
 (segment (start 140.7863 38.1142) (end 140.7863 40.8142) (width 0.2) (layer "F.Cu") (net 36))
 (segment (start 112.0863 39.4142) (end 103.121 39.4142) (width 0.2) (layer "F.Cu") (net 36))
 (segment (start 143.9863 37.3142) (end 143.4863 37.8142) (width 0.2) (layer "F.Cu") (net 36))
 (segment (start 83.7863 40.6642) (end 83.7863 40.9642) (width 0.2) (layer "F.Cu") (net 36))
 (segment (start 65.430014 51.9484) (end 144.3521 51.9484) (width 0.2) (layer "F.Cu") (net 36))
 (segment (start 144.4863 51.8142) (end 144.4863 37.3142) (width 0.2) (layer "F.Cu") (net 36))
 (segment (start 83.7863 41.2642) (end 83.7863 40.9642) (width 0.2) (layer "F.Cu") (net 36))
 (segment (start 140.4863 37.8142) (end 140.7863 38.1142) (width 0.2) (layer "F.Cu") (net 36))
 (segment (start 113.3863 40.7142) (end 112.0863 39.4142) (width 0.2) (layer "F.Cu") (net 36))
 (segment (start 96.4863 46.0489) (end 93.2272 49.308) (width 0.2) (layer "F.Cu") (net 36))
 (segment (start 100.271 42.2642) (end 81.1863 42.2642) (width 0.2) (layer "F.Cu") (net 36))
 (segment (start 88.871 46.0489) (end 83.7863 40.9642) (width 0.2) (layer "F.Cu") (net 36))
 (segment (start 113.3863 41.0142) (end 113.3863 40.7142) (width 0.2) (layer "F.Cu") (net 36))
 (segment (start 137.1863 40.1142) (end 137.1863 40.8142) (width 0.2) (layer "F.Cu") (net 35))
 (segment (start 71.6454 49.708) (end 101.0925 49.708) (width 0.2) (layer "F.Cu") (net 35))
 (segment (start 127.9863 49.708) (end 130.9863 49.708) (width 0.2) (layer "F.Cu") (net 35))
 (segment (start 137.1863 40.8142) (end 137.1863 43.508) (width 0.2) (layer "F.Cu") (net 35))
 (segment (start 71.6454 49.708) (end 127.9863 49.708) (width 0.2) (layer "F.Cu") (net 35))
 (segment (start 68.4863 46.5489) (end 74.6016 46.5489) (width 0.2) (layer "F.Cu") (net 35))
 (segment (start 74.6016 46.5489) (end 80.1863 40.9642) (width 0.2) (layer "F.Cu") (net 35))
 (segment (start 68.4863 46.5489) (end 71.6454 49.708) (width 0.2) (layer "F.Cu") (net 35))
 (segment (start 137.1863 43.508) (end 130.9863 49.708) (width 0.2) (layer "F.Cu") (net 35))
 (segment (start 109.7863 39.8142) (end 109.7863 41.0142) (width 0.2) (layer "F.Cu") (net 35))
 (segment (start 101.0925 49.708) (end 109.7863 41.0142) (width 0.2) (layer "F.Cu") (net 35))
 (segment (start 94.2003 54.2277) (end 93.1557 53.1831) (width 0.2) (layer "F.Cu") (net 27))
 (segment (start 70.0024 57.8303) (end 115.67815 57.8303) (width 0.2) (layer "F.Cu") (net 27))
 (segment (start 93.1557 53.1831) (end 70.0024 53.1831) (width 0.2) (layer "F.Cu") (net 27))
 (segment (start 70.0024 53.1831) (end 70.0024 57.8303) (width 0.2) (layer "F.Cu") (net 27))
 (segment (start 115.67815 57.8303) (end 120.6063 62.75845) (width 0.2) (layer "F.Cu") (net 27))
 (segment (start 149.44085 53.493) (end 127.2723 53.493) (width 0.2) (layer "F.Cu") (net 2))
 (segment (start 97.2277 55.7723) (end 71.8169 55.7723) (width 0.2) (layer "F.Cu") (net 2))
 (segment (start 71.8169 55.7723) (end 70.7723 54.7277) (width 0.2) (layer "F.Cu") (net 2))
 (segment (start 127.2723 53.493) (end 125.39555 55.36975) (width 0.2) (layer "F.Cu") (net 2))
 (segment (start 125.39555 55.36975) (end 99.91435 55.36975) (width 0.2) (layer "F.Cu") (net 2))
 (segment (start 98.7723 54.2277) (end 97.2277 55.7723) (width 0.2) (layer "F.Cu") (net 2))
 (segment (start 99.91435 55.36975) (end 98.7723 54.2277) (width 0.2) (layer "F.Cu") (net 2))
 (segment (start 158.7063 62.75845) (end 149.44085 53.493) (width 0.2) (layer "F.Cu") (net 2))
 (segment (start 121.8904 52.6831) (end 65.9304 52.6831) (width 0.2) (layer "F.Cu") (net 1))
 (segment (start 104.889954 64.14845) (end 107.32055 64.14845) (width 0.2) (layer "F.Cu") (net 1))
 (segment (start 107.429954 64.14845) (end 121.7563 64.14845) (width 0.2) (layer "F.Cu") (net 1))
 (segment (start 103.542646 66.44845) (end 104.2163 65.774796) (width 0.2) (layer "F.Cu") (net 1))
 (segment (start 107.32055 64.14845) (end 107.375252 64.203152) (width 0.2) (layer "F.Cu") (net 1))
 (segment (start 66.1163 63.234796) (end 66.789954 63.90845) (width 0.2) (layer "F.Cu") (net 1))
 (segment (start 122.7003 54.493) (end 122.7003 54.96975) (width 0.2) (layer "F.Cu") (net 1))
 (segment (start 66.789954 63.90845) (end 93.39205 63.90845) (width 0.2) (layer "F.Cu") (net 1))
 (segment (start 104.2163 64.822104) (end 104.889954 64.14845) (width 0.2) (layer "F.Cu") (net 1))
 (segment (start 66.1163 62.522104) (end 66.1163 63.234796) (width 0.2) (layer "F.Cu") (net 1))
 (segment (start 93.39205 63.90845) (end 94.0563 64.5727) (width 0.2) (layer "F.Cu") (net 1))
 (segment (start 65.4304 61.836204) (end 66.1163 62.522104) (width 0.2) (layer "F.Cu") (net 1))
 (segment (start 94.0563 64.5727) (end 94.0563 65.774796) (width 0.2) (layer "F.Cu") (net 1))
 (segment (start 104.2163 65.774796) (end 104.2163 64.822104) (width 0.2) (layer "F.Cu") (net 1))
 (segment (start 94.729954 66.44845) (end 103.542646 66.44845) (width 0.2) (layer "F.Cu") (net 1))
 (segment (start 121.7563 64.14845) (end 123.1463 62.75845) (width 0.2) (layer "F.Cu") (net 1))
 (segment (start 122.7003 53.493) (end 121.8904 52.6831) (width 0.2) (layer "F.Cu") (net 1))
 (segment (start 94.0563 65.774796) (end 94.729954 66.44845) (width 0.2) (layer "F.Cu") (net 1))
 (segment (start 65.9304 52.6831) (end 65.4304 53.1831) (width 0.2) (layer "F.Cu") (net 1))
 (segment (start 65.4304 53.1831) (end 65.4304 61.836204) (width 0.2) (layer "F.Cu") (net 1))
 (segment (start 107.375252 64.203152) (end 107.429954 64.14845) (width 0.2) (layer "F.Cu") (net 1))
 (segment (start 156.9863 40.67845) (end 160.6563 44.34845) (width 0.2) (layer "F.Cu") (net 9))
 (segment (start 149.6963 64.14845) (end 151.0863 62.75845) (width 0.2) (layer "F.Cu") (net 9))
 (segment (start 147.3963 64.822104) (end 148.069954 64.14845) (width 0.2) (layer "F.Cu") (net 9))
 (segment (start 160.6563 44.34845) (end 160.6563 66.6442) (width 0.2) (layer "F.Cu") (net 9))
 (segment (start 160.6563 66.6442) (end 159.6863 67.6142) (width 0.2) (layer "F.Cu") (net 9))
 (segment (start 159.6863 67.6142) (end 149.235704 67.6142) (width 0.2) (layer "F.Cu") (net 9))
 (segment (start 148.069954 64.14845) (end 149.6963 64.14845) (width 0.2) (layer "F.Cu") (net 9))
 (segment (start 149.235704 67.6142) (end 147.3963 65.774796) (width 0.2) (layer "F.Cu") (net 9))
 (segment (start 147.3963 65.774796) (end 147.3963 64.822104) (width 0.2) (layer "F.Cu") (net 9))
 (segment (start 155.32055 64.14845) (end 157.5563 64.14845) (width 0.2) (layer "F.Cu") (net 4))
 (segment (start 155.0163 62.522104) (end 155.0163 63.8442) (width 0.2) (layer "F.Cu") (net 4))
 (segment (start 139.5363 62.2642) (end 140.59205 61.20845) (width 0.2) (layer "F.Cu") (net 4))
 (segment (start 153.702646 61.20845) (end 155.0163 62.522104) (width 0.2) (layer "F.Cu") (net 4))
 (segment (start 155.0163 63.8442) (end 155.32055 64.14845) (width 0.2) (layer "F.Cu") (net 4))
 (segment (start 156.9863 38.13845) (end 161.0563 42.20845) (width 0.2) (layer "F.Cu") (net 4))
 (segment (start 160.2863 68.0142) (end 144.6863 68.0142) (width 0.2) (layer "F.Cu") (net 4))
 (segment (start 161.0563 42.20845) (end 161.0563 67.2442) (width 0.2) (layer "F.Cu") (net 4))
 (segment (start 144.6863 68.0142) (end 144.4863 67.8142) (width 0.2) (layer "F.Cu") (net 4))
 (segment (start 141.815704 67.8142) (end 139.5363 65.534796) (width 0.2) (layer "F.Cu") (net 4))
 (segment (start 139.5363 65.534796) (end 139.5363 62.2642) (width 0.2) (layer "F.Cu") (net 4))
 (segment (start 161.0563 67.2442) (end 160.2863 68.0142) (width 0.2) (layer "F.Cu") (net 4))
 (segment (start 157.5563 64.14845) (end 158.7063 65.29845) (width 0.2) (layer "F.Cu") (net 4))
 (segment (start 144.4863 67.8142) (end 141.815704 67.8142) (width 0.2) (layer "F.Cu") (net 4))
 (segment (start 140.59205 61.20845) (end 153.702646 61.20845) (width 0.2) (layer "F.Cu") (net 4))
 (segment (start 160.2563 66.0442) (end 159.0863 67.2142) (width 0.2) (layer "F.Cu") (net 11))
 (segment (start 159.0863 67.2142) (end 150.46205 67.2142) (width 0.2) (layer "F.Cu") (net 11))
 (segment (start 156.9863 43.21845) (end 160.2563 46.48845) (width 0.2) (layer "F.Cu") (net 11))
 (segment (start 150.46205 67.2142) (end 148.5463 65.29845) (width 0.2) (layer "F.Cu") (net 11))
 (segment (start 160.2563 46.48845) (end 160.2563 66.0442) (width 0.2) (layer "F.Cu") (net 11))
 (segment (start 66.2003 54.7277) (end 73.08105 61.60845) (width 0.2) (layer "F.Cu") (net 29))
 (segment (start 73.08105 61.60845) (end 116.9163 61.60845) (width 0.2) (layer "F.Cu") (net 29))
 (segment (start 116.9163 61.60845) (end 118.0663 62.75845) (width 0.2) (layer "F.Cu") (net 29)))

